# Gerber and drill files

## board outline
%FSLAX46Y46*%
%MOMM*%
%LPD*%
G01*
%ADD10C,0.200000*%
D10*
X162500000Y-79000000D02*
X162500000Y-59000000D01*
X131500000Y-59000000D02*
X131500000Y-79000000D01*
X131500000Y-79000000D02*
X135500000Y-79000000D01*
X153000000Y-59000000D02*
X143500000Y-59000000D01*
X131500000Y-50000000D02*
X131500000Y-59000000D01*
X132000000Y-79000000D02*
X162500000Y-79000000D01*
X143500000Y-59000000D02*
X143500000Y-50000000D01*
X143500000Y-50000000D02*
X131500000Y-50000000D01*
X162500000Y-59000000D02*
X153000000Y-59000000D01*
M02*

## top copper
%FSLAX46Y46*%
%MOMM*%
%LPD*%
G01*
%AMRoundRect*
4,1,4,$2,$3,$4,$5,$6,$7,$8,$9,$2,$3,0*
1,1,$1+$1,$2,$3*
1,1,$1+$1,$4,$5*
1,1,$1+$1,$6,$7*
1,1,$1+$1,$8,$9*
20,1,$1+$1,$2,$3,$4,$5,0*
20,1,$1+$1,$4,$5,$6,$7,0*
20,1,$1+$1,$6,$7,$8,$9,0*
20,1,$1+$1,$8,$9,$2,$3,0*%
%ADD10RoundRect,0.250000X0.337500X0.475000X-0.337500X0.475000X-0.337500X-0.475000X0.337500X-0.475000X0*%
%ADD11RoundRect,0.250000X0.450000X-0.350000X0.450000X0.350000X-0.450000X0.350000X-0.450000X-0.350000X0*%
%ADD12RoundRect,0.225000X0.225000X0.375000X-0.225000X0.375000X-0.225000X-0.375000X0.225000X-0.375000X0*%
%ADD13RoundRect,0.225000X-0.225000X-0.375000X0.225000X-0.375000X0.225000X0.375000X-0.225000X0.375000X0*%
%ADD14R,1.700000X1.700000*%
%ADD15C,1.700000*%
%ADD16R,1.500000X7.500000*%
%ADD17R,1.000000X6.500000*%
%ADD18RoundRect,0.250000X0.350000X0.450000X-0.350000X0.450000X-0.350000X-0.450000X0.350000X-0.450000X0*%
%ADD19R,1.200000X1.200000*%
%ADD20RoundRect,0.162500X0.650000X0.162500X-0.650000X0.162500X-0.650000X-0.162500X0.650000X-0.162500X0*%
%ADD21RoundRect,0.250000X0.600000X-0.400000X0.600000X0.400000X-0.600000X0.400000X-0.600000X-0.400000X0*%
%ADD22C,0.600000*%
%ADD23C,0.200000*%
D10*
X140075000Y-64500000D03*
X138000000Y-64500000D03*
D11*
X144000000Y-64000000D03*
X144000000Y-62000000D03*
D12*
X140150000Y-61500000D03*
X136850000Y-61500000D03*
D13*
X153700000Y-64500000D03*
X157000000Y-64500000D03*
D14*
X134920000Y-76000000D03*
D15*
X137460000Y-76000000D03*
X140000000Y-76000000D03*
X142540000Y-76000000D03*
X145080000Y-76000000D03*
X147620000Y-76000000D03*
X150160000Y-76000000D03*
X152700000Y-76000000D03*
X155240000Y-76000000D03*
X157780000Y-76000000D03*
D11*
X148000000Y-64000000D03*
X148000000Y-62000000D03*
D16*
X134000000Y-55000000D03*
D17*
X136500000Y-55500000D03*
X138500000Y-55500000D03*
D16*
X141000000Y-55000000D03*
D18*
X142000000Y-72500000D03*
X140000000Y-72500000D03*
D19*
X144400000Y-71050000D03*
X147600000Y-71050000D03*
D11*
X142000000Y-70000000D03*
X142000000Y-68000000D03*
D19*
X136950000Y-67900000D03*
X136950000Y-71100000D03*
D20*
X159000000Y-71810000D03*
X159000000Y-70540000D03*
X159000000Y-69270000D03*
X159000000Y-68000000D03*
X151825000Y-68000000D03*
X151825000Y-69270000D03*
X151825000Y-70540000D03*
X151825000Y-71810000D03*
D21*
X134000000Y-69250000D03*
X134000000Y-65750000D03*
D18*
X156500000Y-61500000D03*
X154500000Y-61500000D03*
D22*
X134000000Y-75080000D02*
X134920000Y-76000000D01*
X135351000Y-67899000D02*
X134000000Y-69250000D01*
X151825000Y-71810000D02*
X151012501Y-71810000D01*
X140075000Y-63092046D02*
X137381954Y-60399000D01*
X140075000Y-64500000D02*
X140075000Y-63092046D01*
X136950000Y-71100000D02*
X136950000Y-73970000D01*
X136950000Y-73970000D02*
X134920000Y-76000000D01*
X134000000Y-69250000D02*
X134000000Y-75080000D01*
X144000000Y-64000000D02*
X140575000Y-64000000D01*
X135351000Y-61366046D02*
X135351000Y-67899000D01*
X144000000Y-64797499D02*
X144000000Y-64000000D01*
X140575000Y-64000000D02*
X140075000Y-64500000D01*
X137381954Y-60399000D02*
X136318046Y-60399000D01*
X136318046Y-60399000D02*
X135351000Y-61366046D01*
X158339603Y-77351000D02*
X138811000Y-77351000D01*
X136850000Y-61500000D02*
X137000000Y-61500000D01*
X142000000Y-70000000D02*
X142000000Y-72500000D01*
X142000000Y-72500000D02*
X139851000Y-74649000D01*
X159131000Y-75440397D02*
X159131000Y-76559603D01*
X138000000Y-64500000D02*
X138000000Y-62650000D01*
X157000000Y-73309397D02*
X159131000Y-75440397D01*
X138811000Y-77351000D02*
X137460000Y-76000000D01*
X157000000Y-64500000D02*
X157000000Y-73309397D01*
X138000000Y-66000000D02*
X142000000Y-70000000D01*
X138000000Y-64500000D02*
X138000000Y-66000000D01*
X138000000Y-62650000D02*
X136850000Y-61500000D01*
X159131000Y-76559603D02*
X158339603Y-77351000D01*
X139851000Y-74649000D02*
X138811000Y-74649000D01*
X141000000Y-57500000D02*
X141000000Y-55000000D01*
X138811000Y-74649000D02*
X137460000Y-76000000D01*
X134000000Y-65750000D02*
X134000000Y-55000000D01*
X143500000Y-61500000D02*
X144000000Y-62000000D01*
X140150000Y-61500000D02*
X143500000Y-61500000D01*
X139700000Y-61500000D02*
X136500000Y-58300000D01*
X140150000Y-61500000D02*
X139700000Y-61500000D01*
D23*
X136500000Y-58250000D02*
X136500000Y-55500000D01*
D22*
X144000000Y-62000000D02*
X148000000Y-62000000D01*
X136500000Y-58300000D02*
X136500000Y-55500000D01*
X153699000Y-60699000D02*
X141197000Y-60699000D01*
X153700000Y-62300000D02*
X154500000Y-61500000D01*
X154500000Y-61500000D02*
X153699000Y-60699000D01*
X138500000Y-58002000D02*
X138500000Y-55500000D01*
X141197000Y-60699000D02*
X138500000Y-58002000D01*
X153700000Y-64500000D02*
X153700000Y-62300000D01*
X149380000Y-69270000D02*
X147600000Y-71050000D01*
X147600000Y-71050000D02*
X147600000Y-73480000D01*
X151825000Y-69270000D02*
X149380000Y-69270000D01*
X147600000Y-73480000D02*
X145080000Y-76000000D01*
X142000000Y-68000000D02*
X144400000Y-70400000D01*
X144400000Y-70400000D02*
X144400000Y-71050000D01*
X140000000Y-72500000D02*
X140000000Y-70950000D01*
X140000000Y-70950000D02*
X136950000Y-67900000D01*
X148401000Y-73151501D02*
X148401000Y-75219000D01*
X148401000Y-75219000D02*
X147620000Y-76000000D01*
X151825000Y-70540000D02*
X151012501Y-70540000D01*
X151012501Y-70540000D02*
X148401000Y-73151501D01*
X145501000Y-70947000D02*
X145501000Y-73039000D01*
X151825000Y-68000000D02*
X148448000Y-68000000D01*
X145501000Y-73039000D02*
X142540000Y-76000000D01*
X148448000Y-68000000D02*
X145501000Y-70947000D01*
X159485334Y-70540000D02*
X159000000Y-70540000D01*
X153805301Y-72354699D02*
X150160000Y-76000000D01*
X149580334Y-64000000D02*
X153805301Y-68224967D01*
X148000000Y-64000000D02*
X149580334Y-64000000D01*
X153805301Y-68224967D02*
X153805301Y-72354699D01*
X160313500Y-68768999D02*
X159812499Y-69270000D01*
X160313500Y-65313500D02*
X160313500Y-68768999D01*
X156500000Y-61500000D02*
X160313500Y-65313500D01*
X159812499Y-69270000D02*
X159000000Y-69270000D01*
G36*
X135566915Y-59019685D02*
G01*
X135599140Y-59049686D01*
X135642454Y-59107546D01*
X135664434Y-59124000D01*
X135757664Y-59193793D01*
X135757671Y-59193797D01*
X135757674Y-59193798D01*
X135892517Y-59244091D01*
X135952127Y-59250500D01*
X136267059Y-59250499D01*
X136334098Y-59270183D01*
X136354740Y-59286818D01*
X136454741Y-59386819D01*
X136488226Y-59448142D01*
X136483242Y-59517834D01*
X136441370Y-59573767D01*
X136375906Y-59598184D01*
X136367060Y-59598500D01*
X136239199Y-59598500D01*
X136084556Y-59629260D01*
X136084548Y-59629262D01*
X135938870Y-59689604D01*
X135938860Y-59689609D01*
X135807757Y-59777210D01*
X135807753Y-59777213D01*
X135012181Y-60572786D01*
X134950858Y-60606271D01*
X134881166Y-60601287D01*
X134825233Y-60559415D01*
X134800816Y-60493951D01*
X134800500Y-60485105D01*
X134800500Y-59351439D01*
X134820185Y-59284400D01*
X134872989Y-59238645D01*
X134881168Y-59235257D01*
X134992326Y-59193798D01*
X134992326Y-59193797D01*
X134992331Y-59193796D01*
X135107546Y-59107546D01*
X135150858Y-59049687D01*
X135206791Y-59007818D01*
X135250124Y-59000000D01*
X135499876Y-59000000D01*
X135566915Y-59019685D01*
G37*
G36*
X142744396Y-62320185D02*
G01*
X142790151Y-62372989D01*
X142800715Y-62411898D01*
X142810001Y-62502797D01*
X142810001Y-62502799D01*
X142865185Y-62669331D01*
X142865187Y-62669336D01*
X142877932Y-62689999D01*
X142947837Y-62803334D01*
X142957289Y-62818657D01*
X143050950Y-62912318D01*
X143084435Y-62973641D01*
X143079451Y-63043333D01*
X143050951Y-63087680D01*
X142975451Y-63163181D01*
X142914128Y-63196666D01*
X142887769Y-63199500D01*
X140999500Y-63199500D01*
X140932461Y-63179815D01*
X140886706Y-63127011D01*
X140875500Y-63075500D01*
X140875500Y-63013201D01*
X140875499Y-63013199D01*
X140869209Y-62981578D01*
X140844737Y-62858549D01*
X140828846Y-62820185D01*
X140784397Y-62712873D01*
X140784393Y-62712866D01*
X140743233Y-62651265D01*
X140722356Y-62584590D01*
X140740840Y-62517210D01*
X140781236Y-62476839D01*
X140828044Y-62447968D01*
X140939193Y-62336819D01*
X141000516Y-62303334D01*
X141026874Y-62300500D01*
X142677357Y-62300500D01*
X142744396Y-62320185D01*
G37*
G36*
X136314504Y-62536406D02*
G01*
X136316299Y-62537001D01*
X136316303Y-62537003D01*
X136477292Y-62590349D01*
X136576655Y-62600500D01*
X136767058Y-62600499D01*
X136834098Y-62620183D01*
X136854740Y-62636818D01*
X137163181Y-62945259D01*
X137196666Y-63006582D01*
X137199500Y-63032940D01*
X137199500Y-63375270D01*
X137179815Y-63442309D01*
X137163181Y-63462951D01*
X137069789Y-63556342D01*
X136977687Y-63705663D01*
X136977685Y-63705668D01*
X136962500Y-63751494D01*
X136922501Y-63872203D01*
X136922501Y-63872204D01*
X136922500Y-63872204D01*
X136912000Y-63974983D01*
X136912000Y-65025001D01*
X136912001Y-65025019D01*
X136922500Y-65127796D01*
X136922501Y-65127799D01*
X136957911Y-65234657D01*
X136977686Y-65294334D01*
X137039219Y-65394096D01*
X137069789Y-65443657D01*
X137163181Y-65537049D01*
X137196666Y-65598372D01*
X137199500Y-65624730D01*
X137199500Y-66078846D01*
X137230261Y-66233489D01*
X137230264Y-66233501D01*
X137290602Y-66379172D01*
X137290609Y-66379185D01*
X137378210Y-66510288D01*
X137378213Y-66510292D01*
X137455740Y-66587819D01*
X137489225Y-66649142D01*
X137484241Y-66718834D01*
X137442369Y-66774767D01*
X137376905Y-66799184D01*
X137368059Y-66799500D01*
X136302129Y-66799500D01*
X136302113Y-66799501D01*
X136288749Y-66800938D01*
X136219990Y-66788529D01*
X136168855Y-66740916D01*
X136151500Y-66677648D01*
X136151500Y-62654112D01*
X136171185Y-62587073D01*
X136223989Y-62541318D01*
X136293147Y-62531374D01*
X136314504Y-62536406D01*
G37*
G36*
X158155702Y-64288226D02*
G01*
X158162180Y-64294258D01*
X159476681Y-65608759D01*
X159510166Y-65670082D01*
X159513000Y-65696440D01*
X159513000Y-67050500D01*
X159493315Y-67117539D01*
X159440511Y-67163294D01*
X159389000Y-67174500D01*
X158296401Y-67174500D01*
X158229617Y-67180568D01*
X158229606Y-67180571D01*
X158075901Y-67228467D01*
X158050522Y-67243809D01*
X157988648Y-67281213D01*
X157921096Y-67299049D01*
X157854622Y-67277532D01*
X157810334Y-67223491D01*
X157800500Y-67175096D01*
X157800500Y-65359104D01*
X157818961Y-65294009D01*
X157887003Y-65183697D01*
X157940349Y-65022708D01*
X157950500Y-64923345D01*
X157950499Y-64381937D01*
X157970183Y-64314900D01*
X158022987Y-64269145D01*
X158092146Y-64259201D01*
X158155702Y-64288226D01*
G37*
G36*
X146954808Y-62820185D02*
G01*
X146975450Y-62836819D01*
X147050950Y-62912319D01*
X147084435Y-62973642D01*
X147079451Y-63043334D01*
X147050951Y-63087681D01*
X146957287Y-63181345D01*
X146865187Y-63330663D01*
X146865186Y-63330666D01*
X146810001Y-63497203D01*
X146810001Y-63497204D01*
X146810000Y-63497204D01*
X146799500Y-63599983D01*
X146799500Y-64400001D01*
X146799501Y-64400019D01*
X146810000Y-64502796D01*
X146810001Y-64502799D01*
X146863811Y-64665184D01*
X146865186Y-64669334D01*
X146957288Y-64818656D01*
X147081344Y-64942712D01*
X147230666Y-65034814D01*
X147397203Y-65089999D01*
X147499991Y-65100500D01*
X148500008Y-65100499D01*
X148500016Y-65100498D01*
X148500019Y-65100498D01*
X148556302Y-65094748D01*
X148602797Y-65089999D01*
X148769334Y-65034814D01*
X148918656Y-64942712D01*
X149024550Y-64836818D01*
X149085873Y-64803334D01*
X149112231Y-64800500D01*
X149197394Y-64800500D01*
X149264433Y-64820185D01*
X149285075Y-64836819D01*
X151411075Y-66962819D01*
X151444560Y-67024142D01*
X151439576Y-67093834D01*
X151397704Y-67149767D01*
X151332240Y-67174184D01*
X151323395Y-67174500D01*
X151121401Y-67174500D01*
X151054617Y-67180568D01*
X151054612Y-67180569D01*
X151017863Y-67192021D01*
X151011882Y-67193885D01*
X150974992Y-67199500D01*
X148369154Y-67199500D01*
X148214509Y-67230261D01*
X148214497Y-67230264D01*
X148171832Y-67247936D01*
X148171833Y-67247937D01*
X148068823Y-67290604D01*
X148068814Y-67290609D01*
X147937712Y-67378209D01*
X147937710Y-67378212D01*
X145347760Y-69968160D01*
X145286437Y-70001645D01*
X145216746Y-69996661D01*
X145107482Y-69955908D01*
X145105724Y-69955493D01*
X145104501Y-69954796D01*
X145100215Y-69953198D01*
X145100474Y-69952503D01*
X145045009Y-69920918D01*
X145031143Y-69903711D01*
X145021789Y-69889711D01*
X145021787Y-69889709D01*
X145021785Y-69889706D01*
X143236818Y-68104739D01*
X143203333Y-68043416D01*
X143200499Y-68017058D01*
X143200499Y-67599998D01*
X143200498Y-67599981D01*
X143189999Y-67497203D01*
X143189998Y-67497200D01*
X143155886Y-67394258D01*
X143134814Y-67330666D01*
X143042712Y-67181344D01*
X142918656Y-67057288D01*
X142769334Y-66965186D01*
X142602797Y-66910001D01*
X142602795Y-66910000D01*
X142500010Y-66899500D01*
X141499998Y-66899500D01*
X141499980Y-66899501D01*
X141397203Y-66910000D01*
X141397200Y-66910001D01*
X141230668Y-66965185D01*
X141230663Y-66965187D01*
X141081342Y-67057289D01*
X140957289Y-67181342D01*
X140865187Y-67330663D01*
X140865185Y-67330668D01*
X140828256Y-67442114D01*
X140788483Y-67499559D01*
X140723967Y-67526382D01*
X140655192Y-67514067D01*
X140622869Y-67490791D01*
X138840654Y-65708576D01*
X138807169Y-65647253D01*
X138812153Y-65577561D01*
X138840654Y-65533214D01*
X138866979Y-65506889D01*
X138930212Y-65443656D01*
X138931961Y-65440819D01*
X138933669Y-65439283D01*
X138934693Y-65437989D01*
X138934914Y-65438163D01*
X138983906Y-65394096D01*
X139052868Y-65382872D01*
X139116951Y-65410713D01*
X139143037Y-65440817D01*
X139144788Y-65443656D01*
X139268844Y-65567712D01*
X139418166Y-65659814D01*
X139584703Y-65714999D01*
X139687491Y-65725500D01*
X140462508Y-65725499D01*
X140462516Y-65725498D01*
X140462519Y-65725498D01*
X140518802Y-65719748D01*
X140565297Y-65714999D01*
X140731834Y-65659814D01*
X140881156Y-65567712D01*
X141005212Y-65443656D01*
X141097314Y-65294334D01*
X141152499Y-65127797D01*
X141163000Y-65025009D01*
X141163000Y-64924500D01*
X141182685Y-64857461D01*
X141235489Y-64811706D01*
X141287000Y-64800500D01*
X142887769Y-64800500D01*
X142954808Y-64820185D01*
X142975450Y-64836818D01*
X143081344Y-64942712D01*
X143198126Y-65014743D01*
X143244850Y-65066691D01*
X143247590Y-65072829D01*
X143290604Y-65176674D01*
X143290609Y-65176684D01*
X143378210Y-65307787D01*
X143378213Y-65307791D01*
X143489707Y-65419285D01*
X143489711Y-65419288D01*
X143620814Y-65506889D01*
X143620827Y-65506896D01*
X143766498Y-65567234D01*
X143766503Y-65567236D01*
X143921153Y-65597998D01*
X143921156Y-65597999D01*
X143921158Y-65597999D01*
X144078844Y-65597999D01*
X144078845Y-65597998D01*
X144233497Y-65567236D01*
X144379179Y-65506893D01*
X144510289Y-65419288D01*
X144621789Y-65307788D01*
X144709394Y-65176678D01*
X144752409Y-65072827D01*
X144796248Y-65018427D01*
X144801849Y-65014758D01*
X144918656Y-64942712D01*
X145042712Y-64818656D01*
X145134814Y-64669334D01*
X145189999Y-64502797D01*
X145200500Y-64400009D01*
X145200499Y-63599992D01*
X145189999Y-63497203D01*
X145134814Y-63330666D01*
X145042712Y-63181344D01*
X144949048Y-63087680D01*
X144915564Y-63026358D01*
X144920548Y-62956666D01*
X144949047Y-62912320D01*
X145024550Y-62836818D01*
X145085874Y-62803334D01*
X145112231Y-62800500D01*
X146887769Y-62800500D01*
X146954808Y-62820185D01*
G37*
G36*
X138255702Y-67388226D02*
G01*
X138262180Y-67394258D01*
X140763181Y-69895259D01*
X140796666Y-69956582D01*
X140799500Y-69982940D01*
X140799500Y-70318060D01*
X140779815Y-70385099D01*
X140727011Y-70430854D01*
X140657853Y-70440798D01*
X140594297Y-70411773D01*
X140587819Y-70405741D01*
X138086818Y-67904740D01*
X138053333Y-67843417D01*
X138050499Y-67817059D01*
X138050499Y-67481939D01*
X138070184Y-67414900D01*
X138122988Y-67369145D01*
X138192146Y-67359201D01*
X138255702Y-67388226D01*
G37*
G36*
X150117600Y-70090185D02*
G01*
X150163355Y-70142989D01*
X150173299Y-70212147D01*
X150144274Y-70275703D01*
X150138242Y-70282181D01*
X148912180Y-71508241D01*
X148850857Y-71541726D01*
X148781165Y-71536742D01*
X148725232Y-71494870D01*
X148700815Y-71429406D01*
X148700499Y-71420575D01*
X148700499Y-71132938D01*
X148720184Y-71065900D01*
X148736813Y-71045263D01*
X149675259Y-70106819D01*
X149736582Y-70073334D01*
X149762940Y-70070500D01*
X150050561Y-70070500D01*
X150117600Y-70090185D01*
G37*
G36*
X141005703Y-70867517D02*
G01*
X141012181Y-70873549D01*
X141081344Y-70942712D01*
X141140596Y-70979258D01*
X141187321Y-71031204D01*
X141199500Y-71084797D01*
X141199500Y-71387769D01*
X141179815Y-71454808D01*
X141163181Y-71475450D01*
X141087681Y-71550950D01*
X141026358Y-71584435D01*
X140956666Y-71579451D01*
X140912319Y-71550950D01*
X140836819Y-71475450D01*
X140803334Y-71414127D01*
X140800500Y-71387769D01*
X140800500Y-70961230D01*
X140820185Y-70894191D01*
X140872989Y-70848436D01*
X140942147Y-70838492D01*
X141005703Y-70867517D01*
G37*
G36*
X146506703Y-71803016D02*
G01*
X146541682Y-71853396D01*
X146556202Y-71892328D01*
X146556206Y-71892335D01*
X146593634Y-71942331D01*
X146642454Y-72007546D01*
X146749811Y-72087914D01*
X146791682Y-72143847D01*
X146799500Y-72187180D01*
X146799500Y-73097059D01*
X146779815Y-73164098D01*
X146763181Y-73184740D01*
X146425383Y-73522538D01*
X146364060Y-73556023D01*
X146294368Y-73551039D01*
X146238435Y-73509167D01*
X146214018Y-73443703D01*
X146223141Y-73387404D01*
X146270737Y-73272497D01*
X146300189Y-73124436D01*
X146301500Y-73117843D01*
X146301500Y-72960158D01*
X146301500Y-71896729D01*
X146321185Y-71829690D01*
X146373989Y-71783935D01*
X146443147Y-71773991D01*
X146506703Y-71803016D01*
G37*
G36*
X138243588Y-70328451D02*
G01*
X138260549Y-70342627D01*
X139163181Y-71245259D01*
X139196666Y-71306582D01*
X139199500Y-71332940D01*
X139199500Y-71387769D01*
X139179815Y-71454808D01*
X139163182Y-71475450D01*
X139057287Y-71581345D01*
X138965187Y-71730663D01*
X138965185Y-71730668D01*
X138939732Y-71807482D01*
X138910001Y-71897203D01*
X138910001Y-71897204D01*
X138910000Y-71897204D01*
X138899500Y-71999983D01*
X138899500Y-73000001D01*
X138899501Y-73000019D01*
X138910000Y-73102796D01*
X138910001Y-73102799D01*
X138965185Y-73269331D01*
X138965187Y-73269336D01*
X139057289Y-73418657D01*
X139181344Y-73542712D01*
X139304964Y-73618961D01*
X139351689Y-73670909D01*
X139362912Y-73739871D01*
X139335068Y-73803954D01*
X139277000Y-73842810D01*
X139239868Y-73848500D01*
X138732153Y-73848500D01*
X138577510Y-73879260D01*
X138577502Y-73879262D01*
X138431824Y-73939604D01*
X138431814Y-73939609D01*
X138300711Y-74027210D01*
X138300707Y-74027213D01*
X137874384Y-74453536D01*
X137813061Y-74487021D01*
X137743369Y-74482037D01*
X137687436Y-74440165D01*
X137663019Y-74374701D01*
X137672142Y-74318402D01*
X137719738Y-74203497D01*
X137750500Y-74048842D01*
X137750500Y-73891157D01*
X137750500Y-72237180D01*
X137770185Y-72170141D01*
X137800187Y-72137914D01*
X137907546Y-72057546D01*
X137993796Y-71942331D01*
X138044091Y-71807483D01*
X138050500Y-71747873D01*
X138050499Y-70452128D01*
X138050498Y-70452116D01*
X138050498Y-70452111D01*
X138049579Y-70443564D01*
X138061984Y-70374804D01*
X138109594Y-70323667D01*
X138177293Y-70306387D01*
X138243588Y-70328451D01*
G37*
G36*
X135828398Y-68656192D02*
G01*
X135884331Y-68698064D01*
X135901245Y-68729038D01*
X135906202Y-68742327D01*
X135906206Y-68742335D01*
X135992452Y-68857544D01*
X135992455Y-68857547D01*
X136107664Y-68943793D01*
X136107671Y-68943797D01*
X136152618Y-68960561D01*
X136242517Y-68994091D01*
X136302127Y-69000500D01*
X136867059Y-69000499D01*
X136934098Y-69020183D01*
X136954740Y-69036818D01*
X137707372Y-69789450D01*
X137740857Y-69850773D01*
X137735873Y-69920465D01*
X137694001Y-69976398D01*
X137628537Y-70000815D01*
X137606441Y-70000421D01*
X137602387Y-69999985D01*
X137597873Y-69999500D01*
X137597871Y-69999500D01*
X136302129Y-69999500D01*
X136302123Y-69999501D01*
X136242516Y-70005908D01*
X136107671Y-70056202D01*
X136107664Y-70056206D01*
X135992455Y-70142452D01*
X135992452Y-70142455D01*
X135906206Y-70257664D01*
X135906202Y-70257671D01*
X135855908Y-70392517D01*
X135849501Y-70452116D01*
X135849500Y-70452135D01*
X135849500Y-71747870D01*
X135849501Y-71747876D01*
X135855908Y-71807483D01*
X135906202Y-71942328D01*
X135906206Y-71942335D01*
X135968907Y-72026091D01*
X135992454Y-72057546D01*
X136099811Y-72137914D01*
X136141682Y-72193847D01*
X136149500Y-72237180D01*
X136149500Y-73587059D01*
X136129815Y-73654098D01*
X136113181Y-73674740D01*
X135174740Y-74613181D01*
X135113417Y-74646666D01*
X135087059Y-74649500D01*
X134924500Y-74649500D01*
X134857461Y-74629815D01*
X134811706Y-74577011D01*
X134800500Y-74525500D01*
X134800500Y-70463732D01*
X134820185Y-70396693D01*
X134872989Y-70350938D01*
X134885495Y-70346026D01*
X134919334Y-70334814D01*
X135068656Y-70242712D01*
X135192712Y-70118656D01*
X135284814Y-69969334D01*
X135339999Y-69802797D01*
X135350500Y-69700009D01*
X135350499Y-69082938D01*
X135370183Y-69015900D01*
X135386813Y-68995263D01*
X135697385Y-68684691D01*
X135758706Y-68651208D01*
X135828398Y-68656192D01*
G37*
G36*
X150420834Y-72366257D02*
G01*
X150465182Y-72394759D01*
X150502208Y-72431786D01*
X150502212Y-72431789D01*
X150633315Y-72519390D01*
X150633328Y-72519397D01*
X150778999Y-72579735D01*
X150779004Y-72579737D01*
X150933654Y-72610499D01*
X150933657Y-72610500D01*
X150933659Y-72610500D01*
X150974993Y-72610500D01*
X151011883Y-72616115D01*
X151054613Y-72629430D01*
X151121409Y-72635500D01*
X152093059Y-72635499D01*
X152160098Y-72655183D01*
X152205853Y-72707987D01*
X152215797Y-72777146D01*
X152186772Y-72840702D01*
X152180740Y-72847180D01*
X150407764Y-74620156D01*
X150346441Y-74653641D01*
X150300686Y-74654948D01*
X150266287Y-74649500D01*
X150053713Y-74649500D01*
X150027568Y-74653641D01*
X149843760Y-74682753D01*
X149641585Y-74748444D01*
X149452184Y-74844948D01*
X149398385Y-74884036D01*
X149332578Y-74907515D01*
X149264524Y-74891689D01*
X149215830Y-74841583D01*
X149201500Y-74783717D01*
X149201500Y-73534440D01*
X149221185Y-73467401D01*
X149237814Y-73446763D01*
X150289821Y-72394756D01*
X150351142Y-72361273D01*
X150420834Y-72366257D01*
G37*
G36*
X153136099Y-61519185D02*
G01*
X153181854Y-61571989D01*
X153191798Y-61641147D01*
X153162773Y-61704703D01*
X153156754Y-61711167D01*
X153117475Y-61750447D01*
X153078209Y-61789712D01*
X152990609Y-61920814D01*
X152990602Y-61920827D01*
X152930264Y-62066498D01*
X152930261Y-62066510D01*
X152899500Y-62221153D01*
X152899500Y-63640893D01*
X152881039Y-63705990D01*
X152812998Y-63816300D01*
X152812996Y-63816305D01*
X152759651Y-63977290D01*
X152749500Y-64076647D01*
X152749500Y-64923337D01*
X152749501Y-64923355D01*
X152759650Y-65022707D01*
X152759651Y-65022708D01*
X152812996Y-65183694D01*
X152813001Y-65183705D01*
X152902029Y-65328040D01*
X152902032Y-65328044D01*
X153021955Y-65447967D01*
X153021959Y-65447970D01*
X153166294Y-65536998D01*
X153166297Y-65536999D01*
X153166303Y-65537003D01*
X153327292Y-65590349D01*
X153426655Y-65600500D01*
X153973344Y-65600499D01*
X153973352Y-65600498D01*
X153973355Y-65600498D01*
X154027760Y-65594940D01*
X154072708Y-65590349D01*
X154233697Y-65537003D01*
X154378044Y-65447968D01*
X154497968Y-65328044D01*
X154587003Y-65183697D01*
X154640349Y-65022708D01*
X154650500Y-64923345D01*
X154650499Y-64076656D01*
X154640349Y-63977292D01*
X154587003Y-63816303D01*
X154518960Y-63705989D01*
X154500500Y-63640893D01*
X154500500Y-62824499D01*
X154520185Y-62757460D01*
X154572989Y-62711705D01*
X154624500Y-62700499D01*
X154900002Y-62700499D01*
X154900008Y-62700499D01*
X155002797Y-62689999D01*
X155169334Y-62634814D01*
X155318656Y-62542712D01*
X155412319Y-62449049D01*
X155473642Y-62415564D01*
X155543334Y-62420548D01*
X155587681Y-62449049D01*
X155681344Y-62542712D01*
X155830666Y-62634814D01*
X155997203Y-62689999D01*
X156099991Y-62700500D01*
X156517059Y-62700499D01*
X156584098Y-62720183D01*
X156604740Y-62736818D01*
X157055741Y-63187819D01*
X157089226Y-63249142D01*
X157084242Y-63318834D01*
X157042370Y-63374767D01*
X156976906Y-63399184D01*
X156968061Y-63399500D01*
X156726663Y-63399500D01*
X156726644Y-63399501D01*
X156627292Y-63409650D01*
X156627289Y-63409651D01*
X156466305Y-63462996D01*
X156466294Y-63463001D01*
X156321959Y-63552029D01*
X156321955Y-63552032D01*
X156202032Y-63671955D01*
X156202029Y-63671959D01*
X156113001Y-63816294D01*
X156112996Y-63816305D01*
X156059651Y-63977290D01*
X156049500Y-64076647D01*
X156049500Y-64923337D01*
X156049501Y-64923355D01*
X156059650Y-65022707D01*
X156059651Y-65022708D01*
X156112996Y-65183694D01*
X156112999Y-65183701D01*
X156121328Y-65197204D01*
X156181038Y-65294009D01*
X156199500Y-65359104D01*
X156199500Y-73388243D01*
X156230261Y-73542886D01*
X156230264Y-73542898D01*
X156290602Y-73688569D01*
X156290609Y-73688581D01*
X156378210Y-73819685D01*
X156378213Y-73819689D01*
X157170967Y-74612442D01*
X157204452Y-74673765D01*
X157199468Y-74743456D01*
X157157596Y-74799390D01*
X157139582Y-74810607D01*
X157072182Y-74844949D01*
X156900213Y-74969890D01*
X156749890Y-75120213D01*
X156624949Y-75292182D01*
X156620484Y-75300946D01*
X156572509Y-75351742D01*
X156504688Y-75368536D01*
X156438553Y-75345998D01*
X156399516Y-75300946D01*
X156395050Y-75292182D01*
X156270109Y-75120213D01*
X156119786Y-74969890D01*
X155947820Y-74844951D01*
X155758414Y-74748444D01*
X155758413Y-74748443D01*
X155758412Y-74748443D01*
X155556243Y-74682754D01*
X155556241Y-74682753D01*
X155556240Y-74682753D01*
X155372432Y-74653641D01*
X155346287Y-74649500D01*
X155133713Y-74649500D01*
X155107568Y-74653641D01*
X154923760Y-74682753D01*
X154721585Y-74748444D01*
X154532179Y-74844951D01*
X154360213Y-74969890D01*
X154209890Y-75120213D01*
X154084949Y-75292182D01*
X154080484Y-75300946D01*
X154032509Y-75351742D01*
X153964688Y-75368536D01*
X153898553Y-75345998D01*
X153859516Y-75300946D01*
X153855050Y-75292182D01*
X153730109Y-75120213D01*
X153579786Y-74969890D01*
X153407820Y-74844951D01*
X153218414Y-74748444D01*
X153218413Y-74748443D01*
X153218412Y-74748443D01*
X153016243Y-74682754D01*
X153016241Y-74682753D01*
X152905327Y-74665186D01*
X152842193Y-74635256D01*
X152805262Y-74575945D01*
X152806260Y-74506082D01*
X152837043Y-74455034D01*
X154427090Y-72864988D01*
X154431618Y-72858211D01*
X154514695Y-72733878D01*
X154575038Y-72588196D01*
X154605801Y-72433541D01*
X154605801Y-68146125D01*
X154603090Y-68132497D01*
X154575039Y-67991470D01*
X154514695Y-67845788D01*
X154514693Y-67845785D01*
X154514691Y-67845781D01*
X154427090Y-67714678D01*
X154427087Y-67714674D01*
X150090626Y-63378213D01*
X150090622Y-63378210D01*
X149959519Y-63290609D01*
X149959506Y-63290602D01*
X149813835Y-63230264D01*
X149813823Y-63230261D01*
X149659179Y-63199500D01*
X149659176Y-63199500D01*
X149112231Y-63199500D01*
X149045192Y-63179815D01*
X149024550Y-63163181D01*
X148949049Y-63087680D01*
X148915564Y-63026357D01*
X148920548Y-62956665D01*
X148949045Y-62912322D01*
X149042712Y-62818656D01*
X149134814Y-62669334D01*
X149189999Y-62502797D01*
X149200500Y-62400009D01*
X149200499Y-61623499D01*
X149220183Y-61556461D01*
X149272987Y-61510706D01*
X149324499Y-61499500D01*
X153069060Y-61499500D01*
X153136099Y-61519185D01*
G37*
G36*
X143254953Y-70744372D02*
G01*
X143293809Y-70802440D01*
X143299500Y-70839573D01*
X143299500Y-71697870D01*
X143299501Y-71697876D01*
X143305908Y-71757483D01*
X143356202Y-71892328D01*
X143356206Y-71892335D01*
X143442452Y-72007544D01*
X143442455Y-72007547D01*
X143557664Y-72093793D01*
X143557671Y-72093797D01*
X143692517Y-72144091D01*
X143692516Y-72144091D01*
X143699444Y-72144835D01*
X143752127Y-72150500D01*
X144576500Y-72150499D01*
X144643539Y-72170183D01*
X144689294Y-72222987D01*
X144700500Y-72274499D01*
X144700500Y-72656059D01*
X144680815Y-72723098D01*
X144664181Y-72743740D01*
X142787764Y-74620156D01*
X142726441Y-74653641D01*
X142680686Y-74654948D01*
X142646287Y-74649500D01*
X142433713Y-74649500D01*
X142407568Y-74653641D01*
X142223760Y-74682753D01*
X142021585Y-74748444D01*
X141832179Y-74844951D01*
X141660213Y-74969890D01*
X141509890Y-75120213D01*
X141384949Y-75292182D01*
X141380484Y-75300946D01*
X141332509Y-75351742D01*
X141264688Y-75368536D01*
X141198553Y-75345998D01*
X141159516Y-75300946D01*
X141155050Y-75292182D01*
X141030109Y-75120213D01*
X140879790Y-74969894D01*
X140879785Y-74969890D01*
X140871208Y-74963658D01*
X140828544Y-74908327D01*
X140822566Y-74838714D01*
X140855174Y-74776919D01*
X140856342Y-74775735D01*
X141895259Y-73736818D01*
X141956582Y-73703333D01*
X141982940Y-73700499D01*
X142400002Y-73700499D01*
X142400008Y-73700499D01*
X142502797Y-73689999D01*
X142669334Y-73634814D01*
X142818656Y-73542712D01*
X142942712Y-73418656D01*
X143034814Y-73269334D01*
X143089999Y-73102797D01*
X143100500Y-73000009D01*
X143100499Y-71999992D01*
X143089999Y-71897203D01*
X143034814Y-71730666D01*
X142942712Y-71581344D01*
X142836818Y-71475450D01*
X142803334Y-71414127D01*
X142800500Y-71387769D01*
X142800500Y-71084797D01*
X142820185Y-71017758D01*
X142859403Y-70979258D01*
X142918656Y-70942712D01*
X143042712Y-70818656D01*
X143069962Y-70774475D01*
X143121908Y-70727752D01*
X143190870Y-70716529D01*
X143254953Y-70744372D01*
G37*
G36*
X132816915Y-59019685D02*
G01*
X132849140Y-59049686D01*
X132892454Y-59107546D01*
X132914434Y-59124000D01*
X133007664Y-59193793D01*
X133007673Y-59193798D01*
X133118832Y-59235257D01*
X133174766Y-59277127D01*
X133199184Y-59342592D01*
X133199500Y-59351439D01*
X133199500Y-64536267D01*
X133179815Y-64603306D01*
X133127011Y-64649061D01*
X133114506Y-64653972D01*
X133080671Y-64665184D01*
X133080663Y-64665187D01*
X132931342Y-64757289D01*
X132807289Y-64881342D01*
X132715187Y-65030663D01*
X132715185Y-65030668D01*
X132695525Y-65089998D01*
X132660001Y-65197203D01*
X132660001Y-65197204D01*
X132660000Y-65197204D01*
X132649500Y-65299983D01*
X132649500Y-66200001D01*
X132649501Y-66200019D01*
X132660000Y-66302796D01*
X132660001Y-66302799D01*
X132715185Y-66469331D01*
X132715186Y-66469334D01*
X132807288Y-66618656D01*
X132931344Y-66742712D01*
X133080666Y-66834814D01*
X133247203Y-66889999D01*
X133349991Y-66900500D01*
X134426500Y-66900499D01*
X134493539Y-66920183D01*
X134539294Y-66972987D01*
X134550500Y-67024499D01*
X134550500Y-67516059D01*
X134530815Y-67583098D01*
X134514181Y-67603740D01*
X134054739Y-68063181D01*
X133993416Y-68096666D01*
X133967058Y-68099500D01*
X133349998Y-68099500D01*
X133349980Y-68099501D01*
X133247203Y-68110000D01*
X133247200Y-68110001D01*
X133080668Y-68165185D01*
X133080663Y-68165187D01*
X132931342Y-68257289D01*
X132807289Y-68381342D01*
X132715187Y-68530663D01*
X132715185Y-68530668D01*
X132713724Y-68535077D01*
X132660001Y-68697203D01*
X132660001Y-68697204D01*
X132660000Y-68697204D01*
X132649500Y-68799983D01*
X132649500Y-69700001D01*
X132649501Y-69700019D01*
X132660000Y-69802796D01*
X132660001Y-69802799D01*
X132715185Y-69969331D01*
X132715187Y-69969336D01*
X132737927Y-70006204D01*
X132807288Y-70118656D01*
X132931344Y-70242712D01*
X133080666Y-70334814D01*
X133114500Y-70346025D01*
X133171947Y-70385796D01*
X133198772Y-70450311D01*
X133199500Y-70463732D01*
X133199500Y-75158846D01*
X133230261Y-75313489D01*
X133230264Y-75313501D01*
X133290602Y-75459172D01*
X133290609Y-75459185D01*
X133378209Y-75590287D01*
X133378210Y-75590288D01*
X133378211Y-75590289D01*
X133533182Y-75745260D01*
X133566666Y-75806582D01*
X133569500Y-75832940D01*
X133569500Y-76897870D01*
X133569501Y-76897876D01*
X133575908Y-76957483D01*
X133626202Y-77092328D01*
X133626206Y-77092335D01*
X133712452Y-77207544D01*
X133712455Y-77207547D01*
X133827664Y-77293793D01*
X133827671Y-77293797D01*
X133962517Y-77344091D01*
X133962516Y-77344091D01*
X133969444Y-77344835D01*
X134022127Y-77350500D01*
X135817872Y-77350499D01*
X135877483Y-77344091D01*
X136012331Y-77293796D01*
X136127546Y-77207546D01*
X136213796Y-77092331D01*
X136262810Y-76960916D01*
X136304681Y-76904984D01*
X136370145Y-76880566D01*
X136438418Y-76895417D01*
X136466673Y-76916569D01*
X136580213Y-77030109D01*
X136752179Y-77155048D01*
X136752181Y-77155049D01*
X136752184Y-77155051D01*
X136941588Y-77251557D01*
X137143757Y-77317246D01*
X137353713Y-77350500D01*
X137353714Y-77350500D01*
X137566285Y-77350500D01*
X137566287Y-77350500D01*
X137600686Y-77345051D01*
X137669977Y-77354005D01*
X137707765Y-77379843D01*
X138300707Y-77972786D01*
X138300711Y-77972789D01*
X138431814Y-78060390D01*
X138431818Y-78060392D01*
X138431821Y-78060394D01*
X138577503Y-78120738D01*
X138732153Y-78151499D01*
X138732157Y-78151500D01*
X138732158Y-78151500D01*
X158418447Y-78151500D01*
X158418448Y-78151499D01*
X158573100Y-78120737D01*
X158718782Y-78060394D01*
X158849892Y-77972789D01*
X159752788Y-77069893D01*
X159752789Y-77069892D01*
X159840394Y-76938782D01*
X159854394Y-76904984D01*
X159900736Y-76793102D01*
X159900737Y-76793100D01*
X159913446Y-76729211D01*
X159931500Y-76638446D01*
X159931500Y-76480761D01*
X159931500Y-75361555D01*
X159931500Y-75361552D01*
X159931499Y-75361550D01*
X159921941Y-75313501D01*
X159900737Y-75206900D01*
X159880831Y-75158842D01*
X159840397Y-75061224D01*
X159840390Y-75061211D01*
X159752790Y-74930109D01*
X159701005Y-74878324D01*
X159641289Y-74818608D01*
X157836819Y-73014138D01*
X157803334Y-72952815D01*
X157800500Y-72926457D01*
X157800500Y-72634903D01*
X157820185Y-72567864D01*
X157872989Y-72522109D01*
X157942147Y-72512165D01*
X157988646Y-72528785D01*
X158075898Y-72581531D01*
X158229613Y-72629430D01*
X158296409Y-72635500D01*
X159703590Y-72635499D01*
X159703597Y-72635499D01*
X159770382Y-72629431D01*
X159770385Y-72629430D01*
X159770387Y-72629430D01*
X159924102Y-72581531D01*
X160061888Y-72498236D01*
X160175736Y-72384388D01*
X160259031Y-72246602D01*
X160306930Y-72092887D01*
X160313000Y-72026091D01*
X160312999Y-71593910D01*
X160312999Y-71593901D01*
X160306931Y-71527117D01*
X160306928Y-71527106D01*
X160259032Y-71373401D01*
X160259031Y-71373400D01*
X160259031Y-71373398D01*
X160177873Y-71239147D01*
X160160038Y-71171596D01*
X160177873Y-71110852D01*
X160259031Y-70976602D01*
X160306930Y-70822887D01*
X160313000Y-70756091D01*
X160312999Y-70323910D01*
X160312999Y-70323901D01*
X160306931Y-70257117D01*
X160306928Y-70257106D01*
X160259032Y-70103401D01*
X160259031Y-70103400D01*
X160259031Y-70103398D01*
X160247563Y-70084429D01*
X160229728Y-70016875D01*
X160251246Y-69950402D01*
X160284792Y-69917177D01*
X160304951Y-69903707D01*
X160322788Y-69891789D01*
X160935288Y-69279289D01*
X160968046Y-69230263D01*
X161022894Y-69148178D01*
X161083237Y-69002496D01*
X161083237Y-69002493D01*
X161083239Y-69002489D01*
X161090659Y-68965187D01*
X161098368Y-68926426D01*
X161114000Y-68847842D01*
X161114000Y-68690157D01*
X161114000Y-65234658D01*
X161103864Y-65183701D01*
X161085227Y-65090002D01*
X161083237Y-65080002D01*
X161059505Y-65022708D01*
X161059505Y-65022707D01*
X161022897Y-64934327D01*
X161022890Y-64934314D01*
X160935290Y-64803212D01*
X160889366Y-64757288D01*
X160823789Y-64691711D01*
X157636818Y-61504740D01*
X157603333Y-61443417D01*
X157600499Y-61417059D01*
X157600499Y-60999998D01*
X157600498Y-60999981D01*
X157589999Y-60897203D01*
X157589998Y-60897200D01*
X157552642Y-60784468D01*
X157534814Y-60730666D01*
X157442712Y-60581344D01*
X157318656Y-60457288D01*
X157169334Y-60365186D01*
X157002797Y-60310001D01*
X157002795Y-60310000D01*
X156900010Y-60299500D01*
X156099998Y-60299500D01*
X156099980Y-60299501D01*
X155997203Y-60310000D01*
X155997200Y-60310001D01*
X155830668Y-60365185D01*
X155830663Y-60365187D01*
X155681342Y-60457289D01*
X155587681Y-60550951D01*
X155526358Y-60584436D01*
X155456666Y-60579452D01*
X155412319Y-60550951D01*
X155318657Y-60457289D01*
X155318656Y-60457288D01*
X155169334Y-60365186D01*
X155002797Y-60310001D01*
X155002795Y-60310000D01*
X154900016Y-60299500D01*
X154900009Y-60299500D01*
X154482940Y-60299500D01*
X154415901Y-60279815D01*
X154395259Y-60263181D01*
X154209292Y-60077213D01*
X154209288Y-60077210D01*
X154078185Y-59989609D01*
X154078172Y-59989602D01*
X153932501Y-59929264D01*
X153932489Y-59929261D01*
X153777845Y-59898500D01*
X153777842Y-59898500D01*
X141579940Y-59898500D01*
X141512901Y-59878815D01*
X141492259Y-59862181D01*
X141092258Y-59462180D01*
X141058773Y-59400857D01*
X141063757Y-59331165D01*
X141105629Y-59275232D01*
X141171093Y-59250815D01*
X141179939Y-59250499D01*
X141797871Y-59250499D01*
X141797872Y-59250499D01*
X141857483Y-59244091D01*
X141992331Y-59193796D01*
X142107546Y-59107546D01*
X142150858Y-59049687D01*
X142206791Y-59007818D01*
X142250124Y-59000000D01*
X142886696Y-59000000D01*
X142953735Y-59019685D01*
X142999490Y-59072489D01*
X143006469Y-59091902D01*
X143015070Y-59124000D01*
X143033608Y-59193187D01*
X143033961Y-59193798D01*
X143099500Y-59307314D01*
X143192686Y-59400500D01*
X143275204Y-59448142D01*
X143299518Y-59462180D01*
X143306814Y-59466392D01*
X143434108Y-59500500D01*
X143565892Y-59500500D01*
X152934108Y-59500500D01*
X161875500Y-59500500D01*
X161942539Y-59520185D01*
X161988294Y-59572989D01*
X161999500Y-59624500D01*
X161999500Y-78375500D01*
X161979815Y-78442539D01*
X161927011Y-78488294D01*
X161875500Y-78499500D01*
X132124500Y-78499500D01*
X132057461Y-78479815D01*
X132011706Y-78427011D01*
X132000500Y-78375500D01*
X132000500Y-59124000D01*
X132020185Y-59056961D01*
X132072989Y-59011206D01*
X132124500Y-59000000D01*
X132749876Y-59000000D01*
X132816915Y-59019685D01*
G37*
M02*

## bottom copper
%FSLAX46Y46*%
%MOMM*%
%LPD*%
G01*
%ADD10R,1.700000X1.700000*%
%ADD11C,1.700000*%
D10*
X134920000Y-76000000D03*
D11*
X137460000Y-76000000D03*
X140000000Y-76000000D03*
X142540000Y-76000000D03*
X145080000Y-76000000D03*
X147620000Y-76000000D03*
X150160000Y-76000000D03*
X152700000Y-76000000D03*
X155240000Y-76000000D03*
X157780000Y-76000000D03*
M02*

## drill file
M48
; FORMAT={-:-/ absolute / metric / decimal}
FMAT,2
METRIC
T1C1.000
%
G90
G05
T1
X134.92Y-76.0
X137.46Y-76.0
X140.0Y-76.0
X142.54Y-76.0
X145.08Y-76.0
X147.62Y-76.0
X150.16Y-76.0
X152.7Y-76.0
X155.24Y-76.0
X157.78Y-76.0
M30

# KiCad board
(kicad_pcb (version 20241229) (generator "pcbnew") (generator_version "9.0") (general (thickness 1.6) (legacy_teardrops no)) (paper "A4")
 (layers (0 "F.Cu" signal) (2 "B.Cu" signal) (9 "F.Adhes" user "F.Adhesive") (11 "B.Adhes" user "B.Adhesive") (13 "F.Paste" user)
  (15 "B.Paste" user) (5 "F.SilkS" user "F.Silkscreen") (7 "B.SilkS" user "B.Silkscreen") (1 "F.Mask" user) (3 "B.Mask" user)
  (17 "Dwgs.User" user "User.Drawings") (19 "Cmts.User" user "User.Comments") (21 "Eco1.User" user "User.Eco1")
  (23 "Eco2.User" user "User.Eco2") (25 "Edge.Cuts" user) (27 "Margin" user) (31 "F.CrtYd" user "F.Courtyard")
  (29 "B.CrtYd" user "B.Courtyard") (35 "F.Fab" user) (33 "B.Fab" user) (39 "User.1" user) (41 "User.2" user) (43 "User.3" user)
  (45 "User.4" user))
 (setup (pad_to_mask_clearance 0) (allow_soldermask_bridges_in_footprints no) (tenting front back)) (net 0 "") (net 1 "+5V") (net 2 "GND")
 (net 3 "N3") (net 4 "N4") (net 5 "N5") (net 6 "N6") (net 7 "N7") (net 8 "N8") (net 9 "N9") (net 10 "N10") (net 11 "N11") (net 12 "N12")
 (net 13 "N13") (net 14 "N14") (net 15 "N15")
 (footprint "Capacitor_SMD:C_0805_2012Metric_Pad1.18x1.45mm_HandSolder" (layer "F.Cu") (at 139.0375 64.5 180)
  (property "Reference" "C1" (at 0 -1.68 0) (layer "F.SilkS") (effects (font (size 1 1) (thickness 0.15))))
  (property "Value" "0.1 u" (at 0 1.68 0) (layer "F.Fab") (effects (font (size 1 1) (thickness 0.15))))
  (pad "1" smd roundrect (at -1.0375 0 180) (size 1.175 1.45) (layers "F.Cu" "F.Mask" "F.Paste") (roundrect_rratio 0.212766) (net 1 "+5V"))
  (pad "2" smd roundrect (at 1.0375 0 180) (size 1.175 1.45) (layers "F.Cu" "F.Mask" "F.Paste") (roundrect_rratio 0.212766) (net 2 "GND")))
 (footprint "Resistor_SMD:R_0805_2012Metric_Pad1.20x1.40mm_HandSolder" (layer "F.Cu") (at 144 63 90)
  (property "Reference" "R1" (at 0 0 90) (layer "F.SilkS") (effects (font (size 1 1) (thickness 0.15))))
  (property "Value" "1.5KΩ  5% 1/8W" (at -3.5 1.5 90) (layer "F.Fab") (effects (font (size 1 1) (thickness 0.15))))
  (pad "1" smd roundrect (at -1 0 90) (size 1.2 1.4) (layers "F.Cu" "F.Mask" "F.Paste") (roundrect_rratio 0.208333) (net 1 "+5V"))
  (pad "2" smd roundrect (at 1 0 90) (size 1.2 1.4) (layers "F.Cu" "F.Mask" "F.Paste") (roundrect_rratio 0.208333) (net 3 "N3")))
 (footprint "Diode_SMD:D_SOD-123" (layer "F.Cu") (at 138.5 61.5 180)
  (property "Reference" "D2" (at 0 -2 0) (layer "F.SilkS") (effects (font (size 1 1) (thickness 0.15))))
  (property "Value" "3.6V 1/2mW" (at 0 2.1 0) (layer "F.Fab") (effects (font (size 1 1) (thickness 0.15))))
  (pad "1" smd roundrect (at -1.65 0 180) (size 0.9 1.2) (layers "F.Cu" "F.Mask" "F.Paste") (roundrect_rratio 0.25) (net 3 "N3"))
  (pad "2" smd roundrect (at 1.65 0 180) (size 0.9 1.2) (layers "F.Cu" "F.Mask" "F.Paste") (roundrect_rratio 0.25) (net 2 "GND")))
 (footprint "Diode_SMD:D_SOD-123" (layer "F.Cu") (at 155.35 64.5)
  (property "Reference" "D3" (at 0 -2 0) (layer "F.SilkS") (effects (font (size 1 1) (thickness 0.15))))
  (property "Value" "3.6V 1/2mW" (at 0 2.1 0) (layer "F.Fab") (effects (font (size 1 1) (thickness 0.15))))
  (pad "1" smd roundrect (at -1.65 0) (size 0.9 1.2) (layers "F.Cu" "F.Mask" "F.Paste") (roundrect_rratio 0.25) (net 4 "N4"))
  (pad "2" smd roundrect (at 1.65 0) (size 0.9 1.2) (layers "F.Cu" "F.Mask" "F.Paste") (roundrect_rratio 0.25) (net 2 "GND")))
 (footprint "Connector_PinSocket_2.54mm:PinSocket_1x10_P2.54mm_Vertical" (layer "F.Cu") (at 134.92 76 90)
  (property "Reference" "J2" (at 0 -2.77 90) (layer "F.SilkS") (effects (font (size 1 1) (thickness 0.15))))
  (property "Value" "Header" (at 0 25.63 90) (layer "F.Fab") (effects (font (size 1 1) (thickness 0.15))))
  (pad "1" thru_hole rect (at 0 0 90) (size 1.7 1.7) (drill 1) (layers "*.Cu" "*.Mask") (remove_unused_layers no) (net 1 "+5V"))
  (pad "2" thru_hole circle (at 0 2.54 90) (size 1.7 1.7) (drill 1) (layers "*.Cu" "*.Mask") (remove_unused_layers no) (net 2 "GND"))
  (pad "3" thru_hole circle (at 0 5.08 90) (size 1.7 1.7) (drill 1) (layers "*.Cu" "*.Mask") (remove_unused_layers no) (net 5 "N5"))
  (pad "4" thru_hole circle (at 0 7.62 90) (size 1.7 1.7) (drill 1) (layers "*.Cu" "*.Mask") (remove_unused_layers no) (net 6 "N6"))
  (pad "5" thru_hole circle (at 0 10.16 90) (size 1.7 1.7) (drill 1) (layers "*.Cu" "*.Mask") (remove_unused_layers no) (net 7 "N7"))
  (pad "6" thru_hole circle (at 0 12.7 90) (size 1.7 1.7) (drill 1) (layers "*.Cu" "*.Mask") (remove_unused_layers no) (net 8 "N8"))
  (pad "7" thru_hole circle (at 0 15.24 90) (size 1.7 1.7) (drill 1) (layers "*.Cu" "*.Mask") (remove_unused_layers no) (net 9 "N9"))
  (pad "8" thru_hole circle (at 0 17.78 90) (size 1.7 1.7) (drill 1) (layers "*.Cu" "*.Mask") (remove_unused_layers no) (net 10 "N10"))
  (pad "9" thru_hole circle (at 0 20.32 90) (size 1.7 1.7) (drill 1) (layers "*.Cu" "*.Mask") (remove_unused_layers no) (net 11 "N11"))
  (pad "10" thru_hole circle (at 0 22.86 90) (size 1.7 1.7) (drill 1) (layers "*.Cu" "*.Mask") (remove_unused_layers no) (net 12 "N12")))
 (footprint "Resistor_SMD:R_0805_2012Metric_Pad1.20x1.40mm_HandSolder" (layer "F.Cu") (at 148 63 90)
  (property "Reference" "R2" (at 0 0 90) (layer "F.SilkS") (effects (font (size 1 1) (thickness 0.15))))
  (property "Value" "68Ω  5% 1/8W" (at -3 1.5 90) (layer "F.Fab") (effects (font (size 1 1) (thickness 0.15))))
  (pad "1" smd roundrect (at -1 0 90) (size 1.2 1.4) (layers "F.Cu" "F.Mask" "F.Paste") (roundrect_rratio 0.208333) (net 9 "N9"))
  (pad "2" smd roundrect (at 1 0 90) (size 1.2 1.4) (layers "F.Cu" "F.Mask" "F.Paste") (roundrect_rratio 0.208333) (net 3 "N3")))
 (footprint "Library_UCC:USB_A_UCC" (layer "F.Cu") (at 137.5 55.2 -90)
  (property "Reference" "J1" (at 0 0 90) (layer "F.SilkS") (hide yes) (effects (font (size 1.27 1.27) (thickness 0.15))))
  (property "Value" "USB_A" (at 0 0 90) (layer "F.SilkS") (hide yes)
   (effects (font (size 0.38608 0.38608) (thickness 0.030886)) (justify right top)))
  (pad "1" smd rect (at -0.2 3.5 270) (size 7.5 1.5) (layers "F.Cu" "F.Mask" "F.Paste") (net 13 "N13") (solder_mask_margin 0.1016))
  (pad "2" smd rect (at 0.3 1 270) (size 6.5 1) (layers "F.Cu" "F.Mask" "F.Paste") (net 3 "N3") (solder_mask_margin 0.1016))
  (pad "3" smd rect (at 0.3 -1 270) (size 6.5 1) (layers "F.Cu" "F.Mask" "F.Paste") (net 4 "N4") (solder_mask_margin 0.1016))
  (pad "4" smd rect (at -0.2 -3.5 270) (size 7.5 1.5) (layers "F.Cu" "F.Mask" "F.Paste") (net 2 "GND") (solder_mask_margin 0.1016)))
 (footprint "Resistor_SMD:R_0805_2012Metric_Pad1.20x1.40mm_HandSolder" (layer "F.Cu") (at 141 72.5 180)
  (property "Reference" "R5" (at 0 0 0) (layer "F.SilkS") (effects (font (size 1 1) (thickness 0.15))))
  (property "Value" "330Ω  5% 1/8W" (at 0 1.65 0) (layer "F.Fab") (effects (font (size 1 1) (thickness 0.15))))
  (pad "1" smd roundrect (at -1 0 180) (size 1.2 1.4) (layers "F.Cu" "F.Mask" "F.Paste") (roundrect_rratio 0.208333) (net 2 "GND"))
  (pad "2" smd roundrect (at 1 0 180) (size 1.2 1.4) (layers "F.Cu" "F.Mask" "F.Paste") (roundrect_rratio 0.208333) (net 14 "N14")))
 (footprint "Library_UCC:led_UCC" (layer "F.Cu") (at 146.5 70.6)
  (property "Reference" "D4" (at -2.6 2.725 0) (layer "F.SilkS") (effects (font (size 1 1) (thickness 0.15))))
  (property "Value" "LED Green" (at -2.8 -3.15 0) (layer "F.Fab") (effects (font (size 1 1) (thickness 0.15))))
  (pad "1" smd rect (at -2.1 0.45) (size 1.2 1.2) (layers "F.Cu" "F.Mask" "F.Paste") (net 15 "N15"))
  (pad "2" smd rect (at 1.1 0.45) (size 1.2 1.2) (layers "F.Cu" "F.Mask" "F.Paste") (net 7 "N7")))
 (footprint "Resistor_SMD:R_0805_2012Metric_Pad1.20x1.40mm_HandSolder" (layer "F.Cu") (at 142 69 90)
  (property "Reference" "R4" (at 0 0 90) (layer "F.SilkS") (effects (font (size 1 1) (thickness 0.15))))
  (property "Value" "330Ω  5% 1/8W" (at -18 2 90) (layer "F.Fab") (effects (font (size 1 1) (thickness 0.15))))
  (pad "1" smd roundrect (at -1 0 90) (size 1.2 1.4) (layers "F.Cu" "F.Mask" "F.Paste") (roundrect_rratio 0.208333) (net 2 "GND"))
  (pad "2" smd roundrect (at 1 0 90) (size 1.2 1.4) (layers "F.Cu" "F.Mask" "F.Paste") (roundrect_rratio 0.208333) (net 15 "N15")))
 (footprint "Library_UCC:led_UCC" (layer "F.Cu") (at 137.4 70 -90)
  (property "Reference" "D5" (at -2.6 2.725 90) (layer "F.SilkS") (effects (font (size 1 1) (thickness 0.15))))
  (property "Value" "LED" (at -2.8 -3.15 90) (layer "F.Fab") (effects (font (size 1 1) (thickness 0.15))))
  (pad "1" smd rect (at -2.1 0.45 270) (size 1.2 1.2) (layers "F.Cu" "F.Mask" "F.Paste") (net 14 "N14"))
  (pad "2" smd rect (at 1.1 0.45 270) (size 1.2 1.2) (layers "F.Cu" "F.Mask" "F.Paste") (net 1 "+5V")))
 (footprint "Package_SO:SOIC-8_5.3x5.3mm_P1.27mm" (layer "F.Cu") (at 155.4125 69.905 180)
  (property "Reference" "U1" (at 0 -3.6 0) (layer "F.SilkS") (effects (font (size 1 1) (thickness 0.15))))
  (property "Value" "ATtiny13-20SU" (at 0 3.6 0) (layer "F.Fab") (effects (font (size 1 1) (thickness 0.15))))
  (pad "1" smd roundrect (at -3.5875 -1.905 180) (size 1.625 0.65) (layers "F.Cu" "F.Mask" "F.Paste") (roundrect_rratio 0.25) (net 11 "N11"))
  (pad "2" smd roundrect (at -3.5875 -0.635 180) (size 1.625 0.65) (layers "F.Cu" "F.Mask" "F.Paste") (roundrect_rratio 0.25) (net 9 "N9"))
  (pad "3" smd roundrect (at -3.5875 0.635 180) (size 1.625 0.65) (layers "F.Cu" "F.Mask" "F.Paste") (roundrect_rratio 0.25) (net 10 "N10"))
  (pad "4" smd roundrect (at -3.5875 1.905 180) (size 1.625 0.65) (layers "F.Cu" "F.Mask" "F.Paste") (roundrect_rratio 0.25) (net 2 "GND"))
  (pad "5" smd roundrect (at 3.5875 1.905 180) (size 1.625 0.65) (layers "F.Cu" "F.Mask" "F.Paste") (roundrect_rratio 0.25) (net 6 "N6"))
  (pad "6" smd roundrect (at 3.5875 0.635 180) (size 1.625 0.65) (layers "F.Cu" "F.Mask" "F.Paste") (roundrect_rratio 0.25) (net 7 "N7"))
  (pad "7" smd roundrect (at 3.5875 -0.635 180) (size 1.625 0.65) (layers "F.Cu" "F.Mask" "F.Paste") (roundrect_rratio 0.25) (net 8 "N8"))
  (pad "8" smd roundrect (at 3.5875 -1.905 180) (size 1.625 0.65) (layers "F.Cu" "F.Mask" "F.Paste") (roundrect_rratio 0.25) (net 1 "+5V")))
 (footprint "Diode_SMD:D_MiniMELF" (layer "F.Cu") (at 134 67.5 90)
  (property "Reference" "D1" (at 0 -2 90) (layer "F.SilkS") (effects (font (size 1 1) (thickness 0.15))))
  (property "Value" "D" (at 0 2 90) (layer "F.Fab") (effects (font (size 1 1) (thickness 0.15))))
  (pad "1" smd roundrect (at -1.75 0 90) (size 1.3 1.7) (layers "F.Cu" "F.Mask" "F.Paste") (roundrect_rratio 0.1923076923) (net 1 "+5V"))
  (pad "2" smd roundrect (at 1.75 0 90) (size 1.3 1.7) (layers "F.Cu" "F.Mask" "F.Paste") (roundrect_rratio 0.1923076923) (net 13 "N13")))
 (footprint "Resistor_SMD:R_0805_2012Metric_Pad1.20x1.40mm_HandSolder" (layer "F.Cu") (at 155.5 61.5 180)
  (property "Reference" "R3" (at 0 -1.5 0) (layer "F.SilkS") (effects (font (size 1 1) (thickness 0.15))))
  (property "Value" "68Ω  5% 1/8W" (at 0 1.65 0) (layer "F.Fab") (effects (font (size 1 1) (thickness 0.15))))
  (pad "1" smd roundrect (at -1 0 180) (size 1.2 1.4) (layers "F.Cu" "F.Mask" "F.Paste") (roundrect_rratio 0.208333) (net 10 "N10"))
  (pad "2" smd roundrect (at 1 0 180) (size 1.2 1.4) (layers "F.Cu" "F.Mask" "F.Paste") (roundrect_rratio 0.208333) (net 4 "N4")))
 (gr_line (start 162.5 79) (end 162.5 59) (stroke (width 0.2) (type solid)) (layer "Edge.Cuts"))
 (gr_line (start 131.5 59) (end 131.5 79) (stroke (width 0.2) (type solid)) (layer "Edge.Cuts"))
 (gr_line (start 131.5 79) (end 135.5 79) (stroke (width 0.2) (type solid)) (layer "Edge.Cuts"))
 (gr_line (start 153 59) (end 143.5 59) (stroke (width 0.2) (type solid)) (layer "Edge.Cuts"))
 (gr_line (start 131.5 50) (end 131.5 59) (stroke (width 0.2) (type solid)) (layer "Edge.Cuts"))
 (gr_line (start 132 79) (end 162.5 79) (stroke (width 0.2) (type solid)) (layer "Edge.Cuts"))
 (gr_line (start 143.5 59) (end 143.5 50) (stroke (width 0.2) (type solid)) (layer "Edge.Cuts"))
 (gr_line (start 143.5 50) (end 131.5 50) (stroke (width 0.2) (type solid)) (layer "Edge.Cuts"))
 (gr_line (start 162.5 59) (end 153 59) (stroke (width 0.2) (type solid)) (layer "Edge.Cuts"))
 (segment (start 134 75.08) (end 134.92 76) (width 0.6) (layer "F.Cu") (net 1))
 (segment (start 135.351 67.899) (end 134 69.25) (width 0.6) (layer "F.Cu") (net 1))
 (segment (start 151.825 71.81) (end 151.012501 71.81) (width 0.6) (layer "F.Cu") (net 1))
 (segment (start 140.075 63.092046) (end 137.381954 60.399) (width 0.6) (layer "F.Cu") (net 1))
 (segment (start 140.075 64.5) (end 140.075 63.092046) (width 0.6) (layer "F.Cu") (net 1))
 (segment (start 136.95 71.1) (end 136.95 73.97) (width 0.6) (layer "F.Cu") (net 1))
 (segment (start 136.95 73.97) (end 134.92 76) (width 0.6) (layer "F.Cu") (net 1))
 (segment (start 134 69.25) (end 134 75.08) (width 0.6) (layer "F.Cu") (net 1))
 (segment (start 144 64) (end 140.575 64) (width 0.6) (layer "F.Cu") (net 1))
 (segment (start 135.351 61.366046) (end 135.351 67.899) (width 0.6) (layer "F.Cu") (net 1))
 (segment (start 144 64.797499) (end 144 64) (width 0.6) (layer "F.Cu") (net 1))
 (segment (start 140.575 64) (end 140.075 64.5) (width 0.6) (layer "F.Cu") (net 1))
 (segment (start 137.381954 60.399) (end 136.318046 60.399) (width 0.6) (layer "F.Cu") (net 1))
 (segment (start 136.318046 60.399) (end 135.351 61.366046) (width 0.6) (layer "F.Cu") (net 1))
 (segment (start 158.339603 77.351) (end 138.811 77.351) (width 0.6) (layer "F.Cu") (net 2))
 (segment (start 136.85 61.5) (end 137 61.5) (width 0.6) (layer "F.Cu") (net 2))
 (segment (start 142 70) (end 142 72.5) (width 0.6) (layer "F.Cu") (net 2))
 (segment (start 142 72.5) (end 139.851 74.649) (width 0.6) (layer "F.Cu") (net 2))
 (segment (start 159.131 75.440397) (end 159.131 76.559603) (width 0.6) (layer "F.Cu") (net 2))
 (segment (start 138 64.5) (end 138 62.65) (width 0.6) (layer "F.Cu") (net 2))
 (segment (start 157 73.309397) (end 159.131 75.440397) (width 0.6) (layer "F.Cu") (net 2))
 (segment (start 138.811 77.351) (end 137.46 76) (width 0.6) (layer "F.Cu") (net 2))
 (segment (start 157 64.5) (end 157 73.309397) (width 0.6) (layer "F.Cu") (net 2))
 (segment (start 138 66) (end 142 70) (width 0.6) (layer "F.Cu") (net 2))
 (segment (start 138 64.5) (end 138 66) (width 0.6) (layer "F.Cu") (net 2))
 (segment (start 138 62.65) (end 136.85 61.5) (width 0.6) (layer "F.Cu") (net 2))
 (segment (start 159.131 76.559603) (end 158.339603 77.351) (width 0.6) (layer "F.Cu") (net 2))
 (segment (start 139.851 74.649) (end 138.811 74.649) (width 0.6) (layer "F.Cu") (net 2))
 (segment (start 141 57.5) (end 141 55) (width 0.6) (layer "F.Cu") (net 2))
 (segment (start 138.811 74.649) (end 137.46 76) (width 0.6) (layer "F.Cu") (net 2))
 (segment (start 134 65.75) (end 134 55) (width 0.6) (layer "F.Cu") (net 13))
 (segment (start 143.5 61.5) (end 144 62) (width 0.6) (layer "F.Cu") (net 3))
 (segment (start 140.15 61.5) (end 143.5 61.5) (width 0.6) (layer "F.Cu") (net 3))
 (segment (start 139.7 61.5) (end 136.5 58.3) (width 0.6) (layer "F.Cu") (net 3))
 (segment (start 140.15 61.5) (end 139.7 61.5) (width 0.6) (layer "F.Cu") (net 3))
 (segment (start 136.5 58.25) (end 136.5 55.5) (width 0.2) (layer "F.Cu") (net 3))
 (segment (start 144 62) (end 148 62) (width 0.6) (layer "F.Cu") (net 3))
 (segment (start 136.5 58.3) (end 136.5 55.5) (width 0.6) (layer "F.Cu") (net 3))
 (segment (start 153.699 60.699) (end 141.197 60.699) (width 0.6) (layer "F.Cu") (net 4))
 (segment (start 153.7 62.3) (end 154.5 61.5) (width 0.6) (layer "F.Cu") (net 4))
 (segment (start 154.5 61.5) (end 153.699 60.699) (width 0.6) (layer "F.Cu") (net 4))
 (segment (start 138.5 58.002) (end 138.5 55.5) (width 0.6) (layer "F.Cu") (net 4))
 (segment (start 141.197 60.699) (end 138.5 58.002) (width 0.6) (layer "F.Cu") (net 4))
 (segment (start 153.7 64.5) (end 153.7 62.3) (width 0.6) (layer "F.Cu") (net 4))
 (segment (start 149.38 69.27) (end 147.6 71.05) (width 0.6) (layer "F.Cu") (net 7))
 (segment (start 147.6 71.05) (end 147.6 73.48) (width 0.6) (layer "F.Cu") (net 7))
 (segment (start 151.825 69.27) (end 149.38 69.27) (width 0.6) (layer "F.Cu") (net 7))
 (segment (start 147.6 73.48) (end 145.08 76) (width 0.6) (layer "F.Cu") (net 7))
 (segment (start 142 68) (end 144.4 70.4) (width 0.6) (layer "F.Cu") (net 15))
 (segment (start 144.4 70.4) (end 144.4 71.05) (width 0.6) (layer "F.Cu") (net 15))
 (segment (start 140 72.5) (end 140 70.95) (width 0.6) (layer "F.Cu") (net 14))
 (segment (start 140 70.95) (end 136.95 67.9) (width 0.6) (layer "F.Cu") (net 14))
 (segment (start 148.401 73.151501) (end 148.401 75.219) (width 0.6) (layer "F.Cu") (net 8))
 (segment (start 148.401 75.219) (end 147.62 76) (width 0.6) (layer "F.Cu") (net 8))
 (segment (start 151.825 70.54) (end 151.012501 70.54) (width 0.6) (layer "F.Cu") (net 8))
 (segment (start 151.012501 70.54) (end 148.401 73.151501) (width 0.6) (layer "F.Cu") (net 8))
 (segment (start 145.501 70.947) (end 145.501 73.039) (width 0.6) (layer "F.Cu") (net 6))
 (segment (start 151.825 68) (end 148.448 68) (width 0.6) (layer "F.Cu") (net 6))
 (segment (start 145.501 73.039) (end 142.54 76) (width 0.6) (layer "F.Cu") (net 6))
 (segment (start 148.448 68) (end 145.501 70.947) (width 0.6) (layer "F.Cu") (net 6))
 (segment (start 159.485334 70.54) (end 159 70.54) (width 0.6) (layer "F.Cu") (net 9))
 (segment (start 153.805301 72.354699) (end 150.16 76) (width 0.6) (layer "F.Cu") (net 9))
 (segment (start 149.580334 64) (end 153.805301 68.224967) (width 0.6) (layer "F.Cu") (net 9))
 (segment (start 148 64) (end 149.580334 64) (width 0.6) (layer "F.Cu") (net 9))
 (segment (start 153.805301 68.224967) (end 153.805301 72.354699) (width 0.6) (layer "F.Cu") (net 9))
 (segment (start 160.3135 68.768999) (end 159.812499 69.27) (width 0.6) (layer "F.Cu") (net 10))
 (segment (start 160.3135 65.3135) (end 160.3135 68.768999) (width 0.6) (layer "F.Cu") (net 10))
 (segment (start 156.5 61.5) (end 160.3135 65.3135) (width 0.6) (layer "F.Cu") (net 10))
 (segment (start 159.812499 69.27) (end 159 69.27) (width 0.6) (layer "F.Cu") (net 10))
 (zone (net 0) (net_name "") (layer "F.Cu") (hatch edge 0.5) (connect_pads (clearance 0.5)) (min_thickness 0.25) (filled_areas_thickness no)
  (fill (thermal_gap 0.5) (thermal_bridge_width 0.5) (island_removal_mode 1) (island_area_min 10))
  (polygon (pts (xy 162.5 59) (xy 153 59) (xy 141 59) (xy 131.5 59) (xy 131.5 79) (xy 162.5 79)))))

